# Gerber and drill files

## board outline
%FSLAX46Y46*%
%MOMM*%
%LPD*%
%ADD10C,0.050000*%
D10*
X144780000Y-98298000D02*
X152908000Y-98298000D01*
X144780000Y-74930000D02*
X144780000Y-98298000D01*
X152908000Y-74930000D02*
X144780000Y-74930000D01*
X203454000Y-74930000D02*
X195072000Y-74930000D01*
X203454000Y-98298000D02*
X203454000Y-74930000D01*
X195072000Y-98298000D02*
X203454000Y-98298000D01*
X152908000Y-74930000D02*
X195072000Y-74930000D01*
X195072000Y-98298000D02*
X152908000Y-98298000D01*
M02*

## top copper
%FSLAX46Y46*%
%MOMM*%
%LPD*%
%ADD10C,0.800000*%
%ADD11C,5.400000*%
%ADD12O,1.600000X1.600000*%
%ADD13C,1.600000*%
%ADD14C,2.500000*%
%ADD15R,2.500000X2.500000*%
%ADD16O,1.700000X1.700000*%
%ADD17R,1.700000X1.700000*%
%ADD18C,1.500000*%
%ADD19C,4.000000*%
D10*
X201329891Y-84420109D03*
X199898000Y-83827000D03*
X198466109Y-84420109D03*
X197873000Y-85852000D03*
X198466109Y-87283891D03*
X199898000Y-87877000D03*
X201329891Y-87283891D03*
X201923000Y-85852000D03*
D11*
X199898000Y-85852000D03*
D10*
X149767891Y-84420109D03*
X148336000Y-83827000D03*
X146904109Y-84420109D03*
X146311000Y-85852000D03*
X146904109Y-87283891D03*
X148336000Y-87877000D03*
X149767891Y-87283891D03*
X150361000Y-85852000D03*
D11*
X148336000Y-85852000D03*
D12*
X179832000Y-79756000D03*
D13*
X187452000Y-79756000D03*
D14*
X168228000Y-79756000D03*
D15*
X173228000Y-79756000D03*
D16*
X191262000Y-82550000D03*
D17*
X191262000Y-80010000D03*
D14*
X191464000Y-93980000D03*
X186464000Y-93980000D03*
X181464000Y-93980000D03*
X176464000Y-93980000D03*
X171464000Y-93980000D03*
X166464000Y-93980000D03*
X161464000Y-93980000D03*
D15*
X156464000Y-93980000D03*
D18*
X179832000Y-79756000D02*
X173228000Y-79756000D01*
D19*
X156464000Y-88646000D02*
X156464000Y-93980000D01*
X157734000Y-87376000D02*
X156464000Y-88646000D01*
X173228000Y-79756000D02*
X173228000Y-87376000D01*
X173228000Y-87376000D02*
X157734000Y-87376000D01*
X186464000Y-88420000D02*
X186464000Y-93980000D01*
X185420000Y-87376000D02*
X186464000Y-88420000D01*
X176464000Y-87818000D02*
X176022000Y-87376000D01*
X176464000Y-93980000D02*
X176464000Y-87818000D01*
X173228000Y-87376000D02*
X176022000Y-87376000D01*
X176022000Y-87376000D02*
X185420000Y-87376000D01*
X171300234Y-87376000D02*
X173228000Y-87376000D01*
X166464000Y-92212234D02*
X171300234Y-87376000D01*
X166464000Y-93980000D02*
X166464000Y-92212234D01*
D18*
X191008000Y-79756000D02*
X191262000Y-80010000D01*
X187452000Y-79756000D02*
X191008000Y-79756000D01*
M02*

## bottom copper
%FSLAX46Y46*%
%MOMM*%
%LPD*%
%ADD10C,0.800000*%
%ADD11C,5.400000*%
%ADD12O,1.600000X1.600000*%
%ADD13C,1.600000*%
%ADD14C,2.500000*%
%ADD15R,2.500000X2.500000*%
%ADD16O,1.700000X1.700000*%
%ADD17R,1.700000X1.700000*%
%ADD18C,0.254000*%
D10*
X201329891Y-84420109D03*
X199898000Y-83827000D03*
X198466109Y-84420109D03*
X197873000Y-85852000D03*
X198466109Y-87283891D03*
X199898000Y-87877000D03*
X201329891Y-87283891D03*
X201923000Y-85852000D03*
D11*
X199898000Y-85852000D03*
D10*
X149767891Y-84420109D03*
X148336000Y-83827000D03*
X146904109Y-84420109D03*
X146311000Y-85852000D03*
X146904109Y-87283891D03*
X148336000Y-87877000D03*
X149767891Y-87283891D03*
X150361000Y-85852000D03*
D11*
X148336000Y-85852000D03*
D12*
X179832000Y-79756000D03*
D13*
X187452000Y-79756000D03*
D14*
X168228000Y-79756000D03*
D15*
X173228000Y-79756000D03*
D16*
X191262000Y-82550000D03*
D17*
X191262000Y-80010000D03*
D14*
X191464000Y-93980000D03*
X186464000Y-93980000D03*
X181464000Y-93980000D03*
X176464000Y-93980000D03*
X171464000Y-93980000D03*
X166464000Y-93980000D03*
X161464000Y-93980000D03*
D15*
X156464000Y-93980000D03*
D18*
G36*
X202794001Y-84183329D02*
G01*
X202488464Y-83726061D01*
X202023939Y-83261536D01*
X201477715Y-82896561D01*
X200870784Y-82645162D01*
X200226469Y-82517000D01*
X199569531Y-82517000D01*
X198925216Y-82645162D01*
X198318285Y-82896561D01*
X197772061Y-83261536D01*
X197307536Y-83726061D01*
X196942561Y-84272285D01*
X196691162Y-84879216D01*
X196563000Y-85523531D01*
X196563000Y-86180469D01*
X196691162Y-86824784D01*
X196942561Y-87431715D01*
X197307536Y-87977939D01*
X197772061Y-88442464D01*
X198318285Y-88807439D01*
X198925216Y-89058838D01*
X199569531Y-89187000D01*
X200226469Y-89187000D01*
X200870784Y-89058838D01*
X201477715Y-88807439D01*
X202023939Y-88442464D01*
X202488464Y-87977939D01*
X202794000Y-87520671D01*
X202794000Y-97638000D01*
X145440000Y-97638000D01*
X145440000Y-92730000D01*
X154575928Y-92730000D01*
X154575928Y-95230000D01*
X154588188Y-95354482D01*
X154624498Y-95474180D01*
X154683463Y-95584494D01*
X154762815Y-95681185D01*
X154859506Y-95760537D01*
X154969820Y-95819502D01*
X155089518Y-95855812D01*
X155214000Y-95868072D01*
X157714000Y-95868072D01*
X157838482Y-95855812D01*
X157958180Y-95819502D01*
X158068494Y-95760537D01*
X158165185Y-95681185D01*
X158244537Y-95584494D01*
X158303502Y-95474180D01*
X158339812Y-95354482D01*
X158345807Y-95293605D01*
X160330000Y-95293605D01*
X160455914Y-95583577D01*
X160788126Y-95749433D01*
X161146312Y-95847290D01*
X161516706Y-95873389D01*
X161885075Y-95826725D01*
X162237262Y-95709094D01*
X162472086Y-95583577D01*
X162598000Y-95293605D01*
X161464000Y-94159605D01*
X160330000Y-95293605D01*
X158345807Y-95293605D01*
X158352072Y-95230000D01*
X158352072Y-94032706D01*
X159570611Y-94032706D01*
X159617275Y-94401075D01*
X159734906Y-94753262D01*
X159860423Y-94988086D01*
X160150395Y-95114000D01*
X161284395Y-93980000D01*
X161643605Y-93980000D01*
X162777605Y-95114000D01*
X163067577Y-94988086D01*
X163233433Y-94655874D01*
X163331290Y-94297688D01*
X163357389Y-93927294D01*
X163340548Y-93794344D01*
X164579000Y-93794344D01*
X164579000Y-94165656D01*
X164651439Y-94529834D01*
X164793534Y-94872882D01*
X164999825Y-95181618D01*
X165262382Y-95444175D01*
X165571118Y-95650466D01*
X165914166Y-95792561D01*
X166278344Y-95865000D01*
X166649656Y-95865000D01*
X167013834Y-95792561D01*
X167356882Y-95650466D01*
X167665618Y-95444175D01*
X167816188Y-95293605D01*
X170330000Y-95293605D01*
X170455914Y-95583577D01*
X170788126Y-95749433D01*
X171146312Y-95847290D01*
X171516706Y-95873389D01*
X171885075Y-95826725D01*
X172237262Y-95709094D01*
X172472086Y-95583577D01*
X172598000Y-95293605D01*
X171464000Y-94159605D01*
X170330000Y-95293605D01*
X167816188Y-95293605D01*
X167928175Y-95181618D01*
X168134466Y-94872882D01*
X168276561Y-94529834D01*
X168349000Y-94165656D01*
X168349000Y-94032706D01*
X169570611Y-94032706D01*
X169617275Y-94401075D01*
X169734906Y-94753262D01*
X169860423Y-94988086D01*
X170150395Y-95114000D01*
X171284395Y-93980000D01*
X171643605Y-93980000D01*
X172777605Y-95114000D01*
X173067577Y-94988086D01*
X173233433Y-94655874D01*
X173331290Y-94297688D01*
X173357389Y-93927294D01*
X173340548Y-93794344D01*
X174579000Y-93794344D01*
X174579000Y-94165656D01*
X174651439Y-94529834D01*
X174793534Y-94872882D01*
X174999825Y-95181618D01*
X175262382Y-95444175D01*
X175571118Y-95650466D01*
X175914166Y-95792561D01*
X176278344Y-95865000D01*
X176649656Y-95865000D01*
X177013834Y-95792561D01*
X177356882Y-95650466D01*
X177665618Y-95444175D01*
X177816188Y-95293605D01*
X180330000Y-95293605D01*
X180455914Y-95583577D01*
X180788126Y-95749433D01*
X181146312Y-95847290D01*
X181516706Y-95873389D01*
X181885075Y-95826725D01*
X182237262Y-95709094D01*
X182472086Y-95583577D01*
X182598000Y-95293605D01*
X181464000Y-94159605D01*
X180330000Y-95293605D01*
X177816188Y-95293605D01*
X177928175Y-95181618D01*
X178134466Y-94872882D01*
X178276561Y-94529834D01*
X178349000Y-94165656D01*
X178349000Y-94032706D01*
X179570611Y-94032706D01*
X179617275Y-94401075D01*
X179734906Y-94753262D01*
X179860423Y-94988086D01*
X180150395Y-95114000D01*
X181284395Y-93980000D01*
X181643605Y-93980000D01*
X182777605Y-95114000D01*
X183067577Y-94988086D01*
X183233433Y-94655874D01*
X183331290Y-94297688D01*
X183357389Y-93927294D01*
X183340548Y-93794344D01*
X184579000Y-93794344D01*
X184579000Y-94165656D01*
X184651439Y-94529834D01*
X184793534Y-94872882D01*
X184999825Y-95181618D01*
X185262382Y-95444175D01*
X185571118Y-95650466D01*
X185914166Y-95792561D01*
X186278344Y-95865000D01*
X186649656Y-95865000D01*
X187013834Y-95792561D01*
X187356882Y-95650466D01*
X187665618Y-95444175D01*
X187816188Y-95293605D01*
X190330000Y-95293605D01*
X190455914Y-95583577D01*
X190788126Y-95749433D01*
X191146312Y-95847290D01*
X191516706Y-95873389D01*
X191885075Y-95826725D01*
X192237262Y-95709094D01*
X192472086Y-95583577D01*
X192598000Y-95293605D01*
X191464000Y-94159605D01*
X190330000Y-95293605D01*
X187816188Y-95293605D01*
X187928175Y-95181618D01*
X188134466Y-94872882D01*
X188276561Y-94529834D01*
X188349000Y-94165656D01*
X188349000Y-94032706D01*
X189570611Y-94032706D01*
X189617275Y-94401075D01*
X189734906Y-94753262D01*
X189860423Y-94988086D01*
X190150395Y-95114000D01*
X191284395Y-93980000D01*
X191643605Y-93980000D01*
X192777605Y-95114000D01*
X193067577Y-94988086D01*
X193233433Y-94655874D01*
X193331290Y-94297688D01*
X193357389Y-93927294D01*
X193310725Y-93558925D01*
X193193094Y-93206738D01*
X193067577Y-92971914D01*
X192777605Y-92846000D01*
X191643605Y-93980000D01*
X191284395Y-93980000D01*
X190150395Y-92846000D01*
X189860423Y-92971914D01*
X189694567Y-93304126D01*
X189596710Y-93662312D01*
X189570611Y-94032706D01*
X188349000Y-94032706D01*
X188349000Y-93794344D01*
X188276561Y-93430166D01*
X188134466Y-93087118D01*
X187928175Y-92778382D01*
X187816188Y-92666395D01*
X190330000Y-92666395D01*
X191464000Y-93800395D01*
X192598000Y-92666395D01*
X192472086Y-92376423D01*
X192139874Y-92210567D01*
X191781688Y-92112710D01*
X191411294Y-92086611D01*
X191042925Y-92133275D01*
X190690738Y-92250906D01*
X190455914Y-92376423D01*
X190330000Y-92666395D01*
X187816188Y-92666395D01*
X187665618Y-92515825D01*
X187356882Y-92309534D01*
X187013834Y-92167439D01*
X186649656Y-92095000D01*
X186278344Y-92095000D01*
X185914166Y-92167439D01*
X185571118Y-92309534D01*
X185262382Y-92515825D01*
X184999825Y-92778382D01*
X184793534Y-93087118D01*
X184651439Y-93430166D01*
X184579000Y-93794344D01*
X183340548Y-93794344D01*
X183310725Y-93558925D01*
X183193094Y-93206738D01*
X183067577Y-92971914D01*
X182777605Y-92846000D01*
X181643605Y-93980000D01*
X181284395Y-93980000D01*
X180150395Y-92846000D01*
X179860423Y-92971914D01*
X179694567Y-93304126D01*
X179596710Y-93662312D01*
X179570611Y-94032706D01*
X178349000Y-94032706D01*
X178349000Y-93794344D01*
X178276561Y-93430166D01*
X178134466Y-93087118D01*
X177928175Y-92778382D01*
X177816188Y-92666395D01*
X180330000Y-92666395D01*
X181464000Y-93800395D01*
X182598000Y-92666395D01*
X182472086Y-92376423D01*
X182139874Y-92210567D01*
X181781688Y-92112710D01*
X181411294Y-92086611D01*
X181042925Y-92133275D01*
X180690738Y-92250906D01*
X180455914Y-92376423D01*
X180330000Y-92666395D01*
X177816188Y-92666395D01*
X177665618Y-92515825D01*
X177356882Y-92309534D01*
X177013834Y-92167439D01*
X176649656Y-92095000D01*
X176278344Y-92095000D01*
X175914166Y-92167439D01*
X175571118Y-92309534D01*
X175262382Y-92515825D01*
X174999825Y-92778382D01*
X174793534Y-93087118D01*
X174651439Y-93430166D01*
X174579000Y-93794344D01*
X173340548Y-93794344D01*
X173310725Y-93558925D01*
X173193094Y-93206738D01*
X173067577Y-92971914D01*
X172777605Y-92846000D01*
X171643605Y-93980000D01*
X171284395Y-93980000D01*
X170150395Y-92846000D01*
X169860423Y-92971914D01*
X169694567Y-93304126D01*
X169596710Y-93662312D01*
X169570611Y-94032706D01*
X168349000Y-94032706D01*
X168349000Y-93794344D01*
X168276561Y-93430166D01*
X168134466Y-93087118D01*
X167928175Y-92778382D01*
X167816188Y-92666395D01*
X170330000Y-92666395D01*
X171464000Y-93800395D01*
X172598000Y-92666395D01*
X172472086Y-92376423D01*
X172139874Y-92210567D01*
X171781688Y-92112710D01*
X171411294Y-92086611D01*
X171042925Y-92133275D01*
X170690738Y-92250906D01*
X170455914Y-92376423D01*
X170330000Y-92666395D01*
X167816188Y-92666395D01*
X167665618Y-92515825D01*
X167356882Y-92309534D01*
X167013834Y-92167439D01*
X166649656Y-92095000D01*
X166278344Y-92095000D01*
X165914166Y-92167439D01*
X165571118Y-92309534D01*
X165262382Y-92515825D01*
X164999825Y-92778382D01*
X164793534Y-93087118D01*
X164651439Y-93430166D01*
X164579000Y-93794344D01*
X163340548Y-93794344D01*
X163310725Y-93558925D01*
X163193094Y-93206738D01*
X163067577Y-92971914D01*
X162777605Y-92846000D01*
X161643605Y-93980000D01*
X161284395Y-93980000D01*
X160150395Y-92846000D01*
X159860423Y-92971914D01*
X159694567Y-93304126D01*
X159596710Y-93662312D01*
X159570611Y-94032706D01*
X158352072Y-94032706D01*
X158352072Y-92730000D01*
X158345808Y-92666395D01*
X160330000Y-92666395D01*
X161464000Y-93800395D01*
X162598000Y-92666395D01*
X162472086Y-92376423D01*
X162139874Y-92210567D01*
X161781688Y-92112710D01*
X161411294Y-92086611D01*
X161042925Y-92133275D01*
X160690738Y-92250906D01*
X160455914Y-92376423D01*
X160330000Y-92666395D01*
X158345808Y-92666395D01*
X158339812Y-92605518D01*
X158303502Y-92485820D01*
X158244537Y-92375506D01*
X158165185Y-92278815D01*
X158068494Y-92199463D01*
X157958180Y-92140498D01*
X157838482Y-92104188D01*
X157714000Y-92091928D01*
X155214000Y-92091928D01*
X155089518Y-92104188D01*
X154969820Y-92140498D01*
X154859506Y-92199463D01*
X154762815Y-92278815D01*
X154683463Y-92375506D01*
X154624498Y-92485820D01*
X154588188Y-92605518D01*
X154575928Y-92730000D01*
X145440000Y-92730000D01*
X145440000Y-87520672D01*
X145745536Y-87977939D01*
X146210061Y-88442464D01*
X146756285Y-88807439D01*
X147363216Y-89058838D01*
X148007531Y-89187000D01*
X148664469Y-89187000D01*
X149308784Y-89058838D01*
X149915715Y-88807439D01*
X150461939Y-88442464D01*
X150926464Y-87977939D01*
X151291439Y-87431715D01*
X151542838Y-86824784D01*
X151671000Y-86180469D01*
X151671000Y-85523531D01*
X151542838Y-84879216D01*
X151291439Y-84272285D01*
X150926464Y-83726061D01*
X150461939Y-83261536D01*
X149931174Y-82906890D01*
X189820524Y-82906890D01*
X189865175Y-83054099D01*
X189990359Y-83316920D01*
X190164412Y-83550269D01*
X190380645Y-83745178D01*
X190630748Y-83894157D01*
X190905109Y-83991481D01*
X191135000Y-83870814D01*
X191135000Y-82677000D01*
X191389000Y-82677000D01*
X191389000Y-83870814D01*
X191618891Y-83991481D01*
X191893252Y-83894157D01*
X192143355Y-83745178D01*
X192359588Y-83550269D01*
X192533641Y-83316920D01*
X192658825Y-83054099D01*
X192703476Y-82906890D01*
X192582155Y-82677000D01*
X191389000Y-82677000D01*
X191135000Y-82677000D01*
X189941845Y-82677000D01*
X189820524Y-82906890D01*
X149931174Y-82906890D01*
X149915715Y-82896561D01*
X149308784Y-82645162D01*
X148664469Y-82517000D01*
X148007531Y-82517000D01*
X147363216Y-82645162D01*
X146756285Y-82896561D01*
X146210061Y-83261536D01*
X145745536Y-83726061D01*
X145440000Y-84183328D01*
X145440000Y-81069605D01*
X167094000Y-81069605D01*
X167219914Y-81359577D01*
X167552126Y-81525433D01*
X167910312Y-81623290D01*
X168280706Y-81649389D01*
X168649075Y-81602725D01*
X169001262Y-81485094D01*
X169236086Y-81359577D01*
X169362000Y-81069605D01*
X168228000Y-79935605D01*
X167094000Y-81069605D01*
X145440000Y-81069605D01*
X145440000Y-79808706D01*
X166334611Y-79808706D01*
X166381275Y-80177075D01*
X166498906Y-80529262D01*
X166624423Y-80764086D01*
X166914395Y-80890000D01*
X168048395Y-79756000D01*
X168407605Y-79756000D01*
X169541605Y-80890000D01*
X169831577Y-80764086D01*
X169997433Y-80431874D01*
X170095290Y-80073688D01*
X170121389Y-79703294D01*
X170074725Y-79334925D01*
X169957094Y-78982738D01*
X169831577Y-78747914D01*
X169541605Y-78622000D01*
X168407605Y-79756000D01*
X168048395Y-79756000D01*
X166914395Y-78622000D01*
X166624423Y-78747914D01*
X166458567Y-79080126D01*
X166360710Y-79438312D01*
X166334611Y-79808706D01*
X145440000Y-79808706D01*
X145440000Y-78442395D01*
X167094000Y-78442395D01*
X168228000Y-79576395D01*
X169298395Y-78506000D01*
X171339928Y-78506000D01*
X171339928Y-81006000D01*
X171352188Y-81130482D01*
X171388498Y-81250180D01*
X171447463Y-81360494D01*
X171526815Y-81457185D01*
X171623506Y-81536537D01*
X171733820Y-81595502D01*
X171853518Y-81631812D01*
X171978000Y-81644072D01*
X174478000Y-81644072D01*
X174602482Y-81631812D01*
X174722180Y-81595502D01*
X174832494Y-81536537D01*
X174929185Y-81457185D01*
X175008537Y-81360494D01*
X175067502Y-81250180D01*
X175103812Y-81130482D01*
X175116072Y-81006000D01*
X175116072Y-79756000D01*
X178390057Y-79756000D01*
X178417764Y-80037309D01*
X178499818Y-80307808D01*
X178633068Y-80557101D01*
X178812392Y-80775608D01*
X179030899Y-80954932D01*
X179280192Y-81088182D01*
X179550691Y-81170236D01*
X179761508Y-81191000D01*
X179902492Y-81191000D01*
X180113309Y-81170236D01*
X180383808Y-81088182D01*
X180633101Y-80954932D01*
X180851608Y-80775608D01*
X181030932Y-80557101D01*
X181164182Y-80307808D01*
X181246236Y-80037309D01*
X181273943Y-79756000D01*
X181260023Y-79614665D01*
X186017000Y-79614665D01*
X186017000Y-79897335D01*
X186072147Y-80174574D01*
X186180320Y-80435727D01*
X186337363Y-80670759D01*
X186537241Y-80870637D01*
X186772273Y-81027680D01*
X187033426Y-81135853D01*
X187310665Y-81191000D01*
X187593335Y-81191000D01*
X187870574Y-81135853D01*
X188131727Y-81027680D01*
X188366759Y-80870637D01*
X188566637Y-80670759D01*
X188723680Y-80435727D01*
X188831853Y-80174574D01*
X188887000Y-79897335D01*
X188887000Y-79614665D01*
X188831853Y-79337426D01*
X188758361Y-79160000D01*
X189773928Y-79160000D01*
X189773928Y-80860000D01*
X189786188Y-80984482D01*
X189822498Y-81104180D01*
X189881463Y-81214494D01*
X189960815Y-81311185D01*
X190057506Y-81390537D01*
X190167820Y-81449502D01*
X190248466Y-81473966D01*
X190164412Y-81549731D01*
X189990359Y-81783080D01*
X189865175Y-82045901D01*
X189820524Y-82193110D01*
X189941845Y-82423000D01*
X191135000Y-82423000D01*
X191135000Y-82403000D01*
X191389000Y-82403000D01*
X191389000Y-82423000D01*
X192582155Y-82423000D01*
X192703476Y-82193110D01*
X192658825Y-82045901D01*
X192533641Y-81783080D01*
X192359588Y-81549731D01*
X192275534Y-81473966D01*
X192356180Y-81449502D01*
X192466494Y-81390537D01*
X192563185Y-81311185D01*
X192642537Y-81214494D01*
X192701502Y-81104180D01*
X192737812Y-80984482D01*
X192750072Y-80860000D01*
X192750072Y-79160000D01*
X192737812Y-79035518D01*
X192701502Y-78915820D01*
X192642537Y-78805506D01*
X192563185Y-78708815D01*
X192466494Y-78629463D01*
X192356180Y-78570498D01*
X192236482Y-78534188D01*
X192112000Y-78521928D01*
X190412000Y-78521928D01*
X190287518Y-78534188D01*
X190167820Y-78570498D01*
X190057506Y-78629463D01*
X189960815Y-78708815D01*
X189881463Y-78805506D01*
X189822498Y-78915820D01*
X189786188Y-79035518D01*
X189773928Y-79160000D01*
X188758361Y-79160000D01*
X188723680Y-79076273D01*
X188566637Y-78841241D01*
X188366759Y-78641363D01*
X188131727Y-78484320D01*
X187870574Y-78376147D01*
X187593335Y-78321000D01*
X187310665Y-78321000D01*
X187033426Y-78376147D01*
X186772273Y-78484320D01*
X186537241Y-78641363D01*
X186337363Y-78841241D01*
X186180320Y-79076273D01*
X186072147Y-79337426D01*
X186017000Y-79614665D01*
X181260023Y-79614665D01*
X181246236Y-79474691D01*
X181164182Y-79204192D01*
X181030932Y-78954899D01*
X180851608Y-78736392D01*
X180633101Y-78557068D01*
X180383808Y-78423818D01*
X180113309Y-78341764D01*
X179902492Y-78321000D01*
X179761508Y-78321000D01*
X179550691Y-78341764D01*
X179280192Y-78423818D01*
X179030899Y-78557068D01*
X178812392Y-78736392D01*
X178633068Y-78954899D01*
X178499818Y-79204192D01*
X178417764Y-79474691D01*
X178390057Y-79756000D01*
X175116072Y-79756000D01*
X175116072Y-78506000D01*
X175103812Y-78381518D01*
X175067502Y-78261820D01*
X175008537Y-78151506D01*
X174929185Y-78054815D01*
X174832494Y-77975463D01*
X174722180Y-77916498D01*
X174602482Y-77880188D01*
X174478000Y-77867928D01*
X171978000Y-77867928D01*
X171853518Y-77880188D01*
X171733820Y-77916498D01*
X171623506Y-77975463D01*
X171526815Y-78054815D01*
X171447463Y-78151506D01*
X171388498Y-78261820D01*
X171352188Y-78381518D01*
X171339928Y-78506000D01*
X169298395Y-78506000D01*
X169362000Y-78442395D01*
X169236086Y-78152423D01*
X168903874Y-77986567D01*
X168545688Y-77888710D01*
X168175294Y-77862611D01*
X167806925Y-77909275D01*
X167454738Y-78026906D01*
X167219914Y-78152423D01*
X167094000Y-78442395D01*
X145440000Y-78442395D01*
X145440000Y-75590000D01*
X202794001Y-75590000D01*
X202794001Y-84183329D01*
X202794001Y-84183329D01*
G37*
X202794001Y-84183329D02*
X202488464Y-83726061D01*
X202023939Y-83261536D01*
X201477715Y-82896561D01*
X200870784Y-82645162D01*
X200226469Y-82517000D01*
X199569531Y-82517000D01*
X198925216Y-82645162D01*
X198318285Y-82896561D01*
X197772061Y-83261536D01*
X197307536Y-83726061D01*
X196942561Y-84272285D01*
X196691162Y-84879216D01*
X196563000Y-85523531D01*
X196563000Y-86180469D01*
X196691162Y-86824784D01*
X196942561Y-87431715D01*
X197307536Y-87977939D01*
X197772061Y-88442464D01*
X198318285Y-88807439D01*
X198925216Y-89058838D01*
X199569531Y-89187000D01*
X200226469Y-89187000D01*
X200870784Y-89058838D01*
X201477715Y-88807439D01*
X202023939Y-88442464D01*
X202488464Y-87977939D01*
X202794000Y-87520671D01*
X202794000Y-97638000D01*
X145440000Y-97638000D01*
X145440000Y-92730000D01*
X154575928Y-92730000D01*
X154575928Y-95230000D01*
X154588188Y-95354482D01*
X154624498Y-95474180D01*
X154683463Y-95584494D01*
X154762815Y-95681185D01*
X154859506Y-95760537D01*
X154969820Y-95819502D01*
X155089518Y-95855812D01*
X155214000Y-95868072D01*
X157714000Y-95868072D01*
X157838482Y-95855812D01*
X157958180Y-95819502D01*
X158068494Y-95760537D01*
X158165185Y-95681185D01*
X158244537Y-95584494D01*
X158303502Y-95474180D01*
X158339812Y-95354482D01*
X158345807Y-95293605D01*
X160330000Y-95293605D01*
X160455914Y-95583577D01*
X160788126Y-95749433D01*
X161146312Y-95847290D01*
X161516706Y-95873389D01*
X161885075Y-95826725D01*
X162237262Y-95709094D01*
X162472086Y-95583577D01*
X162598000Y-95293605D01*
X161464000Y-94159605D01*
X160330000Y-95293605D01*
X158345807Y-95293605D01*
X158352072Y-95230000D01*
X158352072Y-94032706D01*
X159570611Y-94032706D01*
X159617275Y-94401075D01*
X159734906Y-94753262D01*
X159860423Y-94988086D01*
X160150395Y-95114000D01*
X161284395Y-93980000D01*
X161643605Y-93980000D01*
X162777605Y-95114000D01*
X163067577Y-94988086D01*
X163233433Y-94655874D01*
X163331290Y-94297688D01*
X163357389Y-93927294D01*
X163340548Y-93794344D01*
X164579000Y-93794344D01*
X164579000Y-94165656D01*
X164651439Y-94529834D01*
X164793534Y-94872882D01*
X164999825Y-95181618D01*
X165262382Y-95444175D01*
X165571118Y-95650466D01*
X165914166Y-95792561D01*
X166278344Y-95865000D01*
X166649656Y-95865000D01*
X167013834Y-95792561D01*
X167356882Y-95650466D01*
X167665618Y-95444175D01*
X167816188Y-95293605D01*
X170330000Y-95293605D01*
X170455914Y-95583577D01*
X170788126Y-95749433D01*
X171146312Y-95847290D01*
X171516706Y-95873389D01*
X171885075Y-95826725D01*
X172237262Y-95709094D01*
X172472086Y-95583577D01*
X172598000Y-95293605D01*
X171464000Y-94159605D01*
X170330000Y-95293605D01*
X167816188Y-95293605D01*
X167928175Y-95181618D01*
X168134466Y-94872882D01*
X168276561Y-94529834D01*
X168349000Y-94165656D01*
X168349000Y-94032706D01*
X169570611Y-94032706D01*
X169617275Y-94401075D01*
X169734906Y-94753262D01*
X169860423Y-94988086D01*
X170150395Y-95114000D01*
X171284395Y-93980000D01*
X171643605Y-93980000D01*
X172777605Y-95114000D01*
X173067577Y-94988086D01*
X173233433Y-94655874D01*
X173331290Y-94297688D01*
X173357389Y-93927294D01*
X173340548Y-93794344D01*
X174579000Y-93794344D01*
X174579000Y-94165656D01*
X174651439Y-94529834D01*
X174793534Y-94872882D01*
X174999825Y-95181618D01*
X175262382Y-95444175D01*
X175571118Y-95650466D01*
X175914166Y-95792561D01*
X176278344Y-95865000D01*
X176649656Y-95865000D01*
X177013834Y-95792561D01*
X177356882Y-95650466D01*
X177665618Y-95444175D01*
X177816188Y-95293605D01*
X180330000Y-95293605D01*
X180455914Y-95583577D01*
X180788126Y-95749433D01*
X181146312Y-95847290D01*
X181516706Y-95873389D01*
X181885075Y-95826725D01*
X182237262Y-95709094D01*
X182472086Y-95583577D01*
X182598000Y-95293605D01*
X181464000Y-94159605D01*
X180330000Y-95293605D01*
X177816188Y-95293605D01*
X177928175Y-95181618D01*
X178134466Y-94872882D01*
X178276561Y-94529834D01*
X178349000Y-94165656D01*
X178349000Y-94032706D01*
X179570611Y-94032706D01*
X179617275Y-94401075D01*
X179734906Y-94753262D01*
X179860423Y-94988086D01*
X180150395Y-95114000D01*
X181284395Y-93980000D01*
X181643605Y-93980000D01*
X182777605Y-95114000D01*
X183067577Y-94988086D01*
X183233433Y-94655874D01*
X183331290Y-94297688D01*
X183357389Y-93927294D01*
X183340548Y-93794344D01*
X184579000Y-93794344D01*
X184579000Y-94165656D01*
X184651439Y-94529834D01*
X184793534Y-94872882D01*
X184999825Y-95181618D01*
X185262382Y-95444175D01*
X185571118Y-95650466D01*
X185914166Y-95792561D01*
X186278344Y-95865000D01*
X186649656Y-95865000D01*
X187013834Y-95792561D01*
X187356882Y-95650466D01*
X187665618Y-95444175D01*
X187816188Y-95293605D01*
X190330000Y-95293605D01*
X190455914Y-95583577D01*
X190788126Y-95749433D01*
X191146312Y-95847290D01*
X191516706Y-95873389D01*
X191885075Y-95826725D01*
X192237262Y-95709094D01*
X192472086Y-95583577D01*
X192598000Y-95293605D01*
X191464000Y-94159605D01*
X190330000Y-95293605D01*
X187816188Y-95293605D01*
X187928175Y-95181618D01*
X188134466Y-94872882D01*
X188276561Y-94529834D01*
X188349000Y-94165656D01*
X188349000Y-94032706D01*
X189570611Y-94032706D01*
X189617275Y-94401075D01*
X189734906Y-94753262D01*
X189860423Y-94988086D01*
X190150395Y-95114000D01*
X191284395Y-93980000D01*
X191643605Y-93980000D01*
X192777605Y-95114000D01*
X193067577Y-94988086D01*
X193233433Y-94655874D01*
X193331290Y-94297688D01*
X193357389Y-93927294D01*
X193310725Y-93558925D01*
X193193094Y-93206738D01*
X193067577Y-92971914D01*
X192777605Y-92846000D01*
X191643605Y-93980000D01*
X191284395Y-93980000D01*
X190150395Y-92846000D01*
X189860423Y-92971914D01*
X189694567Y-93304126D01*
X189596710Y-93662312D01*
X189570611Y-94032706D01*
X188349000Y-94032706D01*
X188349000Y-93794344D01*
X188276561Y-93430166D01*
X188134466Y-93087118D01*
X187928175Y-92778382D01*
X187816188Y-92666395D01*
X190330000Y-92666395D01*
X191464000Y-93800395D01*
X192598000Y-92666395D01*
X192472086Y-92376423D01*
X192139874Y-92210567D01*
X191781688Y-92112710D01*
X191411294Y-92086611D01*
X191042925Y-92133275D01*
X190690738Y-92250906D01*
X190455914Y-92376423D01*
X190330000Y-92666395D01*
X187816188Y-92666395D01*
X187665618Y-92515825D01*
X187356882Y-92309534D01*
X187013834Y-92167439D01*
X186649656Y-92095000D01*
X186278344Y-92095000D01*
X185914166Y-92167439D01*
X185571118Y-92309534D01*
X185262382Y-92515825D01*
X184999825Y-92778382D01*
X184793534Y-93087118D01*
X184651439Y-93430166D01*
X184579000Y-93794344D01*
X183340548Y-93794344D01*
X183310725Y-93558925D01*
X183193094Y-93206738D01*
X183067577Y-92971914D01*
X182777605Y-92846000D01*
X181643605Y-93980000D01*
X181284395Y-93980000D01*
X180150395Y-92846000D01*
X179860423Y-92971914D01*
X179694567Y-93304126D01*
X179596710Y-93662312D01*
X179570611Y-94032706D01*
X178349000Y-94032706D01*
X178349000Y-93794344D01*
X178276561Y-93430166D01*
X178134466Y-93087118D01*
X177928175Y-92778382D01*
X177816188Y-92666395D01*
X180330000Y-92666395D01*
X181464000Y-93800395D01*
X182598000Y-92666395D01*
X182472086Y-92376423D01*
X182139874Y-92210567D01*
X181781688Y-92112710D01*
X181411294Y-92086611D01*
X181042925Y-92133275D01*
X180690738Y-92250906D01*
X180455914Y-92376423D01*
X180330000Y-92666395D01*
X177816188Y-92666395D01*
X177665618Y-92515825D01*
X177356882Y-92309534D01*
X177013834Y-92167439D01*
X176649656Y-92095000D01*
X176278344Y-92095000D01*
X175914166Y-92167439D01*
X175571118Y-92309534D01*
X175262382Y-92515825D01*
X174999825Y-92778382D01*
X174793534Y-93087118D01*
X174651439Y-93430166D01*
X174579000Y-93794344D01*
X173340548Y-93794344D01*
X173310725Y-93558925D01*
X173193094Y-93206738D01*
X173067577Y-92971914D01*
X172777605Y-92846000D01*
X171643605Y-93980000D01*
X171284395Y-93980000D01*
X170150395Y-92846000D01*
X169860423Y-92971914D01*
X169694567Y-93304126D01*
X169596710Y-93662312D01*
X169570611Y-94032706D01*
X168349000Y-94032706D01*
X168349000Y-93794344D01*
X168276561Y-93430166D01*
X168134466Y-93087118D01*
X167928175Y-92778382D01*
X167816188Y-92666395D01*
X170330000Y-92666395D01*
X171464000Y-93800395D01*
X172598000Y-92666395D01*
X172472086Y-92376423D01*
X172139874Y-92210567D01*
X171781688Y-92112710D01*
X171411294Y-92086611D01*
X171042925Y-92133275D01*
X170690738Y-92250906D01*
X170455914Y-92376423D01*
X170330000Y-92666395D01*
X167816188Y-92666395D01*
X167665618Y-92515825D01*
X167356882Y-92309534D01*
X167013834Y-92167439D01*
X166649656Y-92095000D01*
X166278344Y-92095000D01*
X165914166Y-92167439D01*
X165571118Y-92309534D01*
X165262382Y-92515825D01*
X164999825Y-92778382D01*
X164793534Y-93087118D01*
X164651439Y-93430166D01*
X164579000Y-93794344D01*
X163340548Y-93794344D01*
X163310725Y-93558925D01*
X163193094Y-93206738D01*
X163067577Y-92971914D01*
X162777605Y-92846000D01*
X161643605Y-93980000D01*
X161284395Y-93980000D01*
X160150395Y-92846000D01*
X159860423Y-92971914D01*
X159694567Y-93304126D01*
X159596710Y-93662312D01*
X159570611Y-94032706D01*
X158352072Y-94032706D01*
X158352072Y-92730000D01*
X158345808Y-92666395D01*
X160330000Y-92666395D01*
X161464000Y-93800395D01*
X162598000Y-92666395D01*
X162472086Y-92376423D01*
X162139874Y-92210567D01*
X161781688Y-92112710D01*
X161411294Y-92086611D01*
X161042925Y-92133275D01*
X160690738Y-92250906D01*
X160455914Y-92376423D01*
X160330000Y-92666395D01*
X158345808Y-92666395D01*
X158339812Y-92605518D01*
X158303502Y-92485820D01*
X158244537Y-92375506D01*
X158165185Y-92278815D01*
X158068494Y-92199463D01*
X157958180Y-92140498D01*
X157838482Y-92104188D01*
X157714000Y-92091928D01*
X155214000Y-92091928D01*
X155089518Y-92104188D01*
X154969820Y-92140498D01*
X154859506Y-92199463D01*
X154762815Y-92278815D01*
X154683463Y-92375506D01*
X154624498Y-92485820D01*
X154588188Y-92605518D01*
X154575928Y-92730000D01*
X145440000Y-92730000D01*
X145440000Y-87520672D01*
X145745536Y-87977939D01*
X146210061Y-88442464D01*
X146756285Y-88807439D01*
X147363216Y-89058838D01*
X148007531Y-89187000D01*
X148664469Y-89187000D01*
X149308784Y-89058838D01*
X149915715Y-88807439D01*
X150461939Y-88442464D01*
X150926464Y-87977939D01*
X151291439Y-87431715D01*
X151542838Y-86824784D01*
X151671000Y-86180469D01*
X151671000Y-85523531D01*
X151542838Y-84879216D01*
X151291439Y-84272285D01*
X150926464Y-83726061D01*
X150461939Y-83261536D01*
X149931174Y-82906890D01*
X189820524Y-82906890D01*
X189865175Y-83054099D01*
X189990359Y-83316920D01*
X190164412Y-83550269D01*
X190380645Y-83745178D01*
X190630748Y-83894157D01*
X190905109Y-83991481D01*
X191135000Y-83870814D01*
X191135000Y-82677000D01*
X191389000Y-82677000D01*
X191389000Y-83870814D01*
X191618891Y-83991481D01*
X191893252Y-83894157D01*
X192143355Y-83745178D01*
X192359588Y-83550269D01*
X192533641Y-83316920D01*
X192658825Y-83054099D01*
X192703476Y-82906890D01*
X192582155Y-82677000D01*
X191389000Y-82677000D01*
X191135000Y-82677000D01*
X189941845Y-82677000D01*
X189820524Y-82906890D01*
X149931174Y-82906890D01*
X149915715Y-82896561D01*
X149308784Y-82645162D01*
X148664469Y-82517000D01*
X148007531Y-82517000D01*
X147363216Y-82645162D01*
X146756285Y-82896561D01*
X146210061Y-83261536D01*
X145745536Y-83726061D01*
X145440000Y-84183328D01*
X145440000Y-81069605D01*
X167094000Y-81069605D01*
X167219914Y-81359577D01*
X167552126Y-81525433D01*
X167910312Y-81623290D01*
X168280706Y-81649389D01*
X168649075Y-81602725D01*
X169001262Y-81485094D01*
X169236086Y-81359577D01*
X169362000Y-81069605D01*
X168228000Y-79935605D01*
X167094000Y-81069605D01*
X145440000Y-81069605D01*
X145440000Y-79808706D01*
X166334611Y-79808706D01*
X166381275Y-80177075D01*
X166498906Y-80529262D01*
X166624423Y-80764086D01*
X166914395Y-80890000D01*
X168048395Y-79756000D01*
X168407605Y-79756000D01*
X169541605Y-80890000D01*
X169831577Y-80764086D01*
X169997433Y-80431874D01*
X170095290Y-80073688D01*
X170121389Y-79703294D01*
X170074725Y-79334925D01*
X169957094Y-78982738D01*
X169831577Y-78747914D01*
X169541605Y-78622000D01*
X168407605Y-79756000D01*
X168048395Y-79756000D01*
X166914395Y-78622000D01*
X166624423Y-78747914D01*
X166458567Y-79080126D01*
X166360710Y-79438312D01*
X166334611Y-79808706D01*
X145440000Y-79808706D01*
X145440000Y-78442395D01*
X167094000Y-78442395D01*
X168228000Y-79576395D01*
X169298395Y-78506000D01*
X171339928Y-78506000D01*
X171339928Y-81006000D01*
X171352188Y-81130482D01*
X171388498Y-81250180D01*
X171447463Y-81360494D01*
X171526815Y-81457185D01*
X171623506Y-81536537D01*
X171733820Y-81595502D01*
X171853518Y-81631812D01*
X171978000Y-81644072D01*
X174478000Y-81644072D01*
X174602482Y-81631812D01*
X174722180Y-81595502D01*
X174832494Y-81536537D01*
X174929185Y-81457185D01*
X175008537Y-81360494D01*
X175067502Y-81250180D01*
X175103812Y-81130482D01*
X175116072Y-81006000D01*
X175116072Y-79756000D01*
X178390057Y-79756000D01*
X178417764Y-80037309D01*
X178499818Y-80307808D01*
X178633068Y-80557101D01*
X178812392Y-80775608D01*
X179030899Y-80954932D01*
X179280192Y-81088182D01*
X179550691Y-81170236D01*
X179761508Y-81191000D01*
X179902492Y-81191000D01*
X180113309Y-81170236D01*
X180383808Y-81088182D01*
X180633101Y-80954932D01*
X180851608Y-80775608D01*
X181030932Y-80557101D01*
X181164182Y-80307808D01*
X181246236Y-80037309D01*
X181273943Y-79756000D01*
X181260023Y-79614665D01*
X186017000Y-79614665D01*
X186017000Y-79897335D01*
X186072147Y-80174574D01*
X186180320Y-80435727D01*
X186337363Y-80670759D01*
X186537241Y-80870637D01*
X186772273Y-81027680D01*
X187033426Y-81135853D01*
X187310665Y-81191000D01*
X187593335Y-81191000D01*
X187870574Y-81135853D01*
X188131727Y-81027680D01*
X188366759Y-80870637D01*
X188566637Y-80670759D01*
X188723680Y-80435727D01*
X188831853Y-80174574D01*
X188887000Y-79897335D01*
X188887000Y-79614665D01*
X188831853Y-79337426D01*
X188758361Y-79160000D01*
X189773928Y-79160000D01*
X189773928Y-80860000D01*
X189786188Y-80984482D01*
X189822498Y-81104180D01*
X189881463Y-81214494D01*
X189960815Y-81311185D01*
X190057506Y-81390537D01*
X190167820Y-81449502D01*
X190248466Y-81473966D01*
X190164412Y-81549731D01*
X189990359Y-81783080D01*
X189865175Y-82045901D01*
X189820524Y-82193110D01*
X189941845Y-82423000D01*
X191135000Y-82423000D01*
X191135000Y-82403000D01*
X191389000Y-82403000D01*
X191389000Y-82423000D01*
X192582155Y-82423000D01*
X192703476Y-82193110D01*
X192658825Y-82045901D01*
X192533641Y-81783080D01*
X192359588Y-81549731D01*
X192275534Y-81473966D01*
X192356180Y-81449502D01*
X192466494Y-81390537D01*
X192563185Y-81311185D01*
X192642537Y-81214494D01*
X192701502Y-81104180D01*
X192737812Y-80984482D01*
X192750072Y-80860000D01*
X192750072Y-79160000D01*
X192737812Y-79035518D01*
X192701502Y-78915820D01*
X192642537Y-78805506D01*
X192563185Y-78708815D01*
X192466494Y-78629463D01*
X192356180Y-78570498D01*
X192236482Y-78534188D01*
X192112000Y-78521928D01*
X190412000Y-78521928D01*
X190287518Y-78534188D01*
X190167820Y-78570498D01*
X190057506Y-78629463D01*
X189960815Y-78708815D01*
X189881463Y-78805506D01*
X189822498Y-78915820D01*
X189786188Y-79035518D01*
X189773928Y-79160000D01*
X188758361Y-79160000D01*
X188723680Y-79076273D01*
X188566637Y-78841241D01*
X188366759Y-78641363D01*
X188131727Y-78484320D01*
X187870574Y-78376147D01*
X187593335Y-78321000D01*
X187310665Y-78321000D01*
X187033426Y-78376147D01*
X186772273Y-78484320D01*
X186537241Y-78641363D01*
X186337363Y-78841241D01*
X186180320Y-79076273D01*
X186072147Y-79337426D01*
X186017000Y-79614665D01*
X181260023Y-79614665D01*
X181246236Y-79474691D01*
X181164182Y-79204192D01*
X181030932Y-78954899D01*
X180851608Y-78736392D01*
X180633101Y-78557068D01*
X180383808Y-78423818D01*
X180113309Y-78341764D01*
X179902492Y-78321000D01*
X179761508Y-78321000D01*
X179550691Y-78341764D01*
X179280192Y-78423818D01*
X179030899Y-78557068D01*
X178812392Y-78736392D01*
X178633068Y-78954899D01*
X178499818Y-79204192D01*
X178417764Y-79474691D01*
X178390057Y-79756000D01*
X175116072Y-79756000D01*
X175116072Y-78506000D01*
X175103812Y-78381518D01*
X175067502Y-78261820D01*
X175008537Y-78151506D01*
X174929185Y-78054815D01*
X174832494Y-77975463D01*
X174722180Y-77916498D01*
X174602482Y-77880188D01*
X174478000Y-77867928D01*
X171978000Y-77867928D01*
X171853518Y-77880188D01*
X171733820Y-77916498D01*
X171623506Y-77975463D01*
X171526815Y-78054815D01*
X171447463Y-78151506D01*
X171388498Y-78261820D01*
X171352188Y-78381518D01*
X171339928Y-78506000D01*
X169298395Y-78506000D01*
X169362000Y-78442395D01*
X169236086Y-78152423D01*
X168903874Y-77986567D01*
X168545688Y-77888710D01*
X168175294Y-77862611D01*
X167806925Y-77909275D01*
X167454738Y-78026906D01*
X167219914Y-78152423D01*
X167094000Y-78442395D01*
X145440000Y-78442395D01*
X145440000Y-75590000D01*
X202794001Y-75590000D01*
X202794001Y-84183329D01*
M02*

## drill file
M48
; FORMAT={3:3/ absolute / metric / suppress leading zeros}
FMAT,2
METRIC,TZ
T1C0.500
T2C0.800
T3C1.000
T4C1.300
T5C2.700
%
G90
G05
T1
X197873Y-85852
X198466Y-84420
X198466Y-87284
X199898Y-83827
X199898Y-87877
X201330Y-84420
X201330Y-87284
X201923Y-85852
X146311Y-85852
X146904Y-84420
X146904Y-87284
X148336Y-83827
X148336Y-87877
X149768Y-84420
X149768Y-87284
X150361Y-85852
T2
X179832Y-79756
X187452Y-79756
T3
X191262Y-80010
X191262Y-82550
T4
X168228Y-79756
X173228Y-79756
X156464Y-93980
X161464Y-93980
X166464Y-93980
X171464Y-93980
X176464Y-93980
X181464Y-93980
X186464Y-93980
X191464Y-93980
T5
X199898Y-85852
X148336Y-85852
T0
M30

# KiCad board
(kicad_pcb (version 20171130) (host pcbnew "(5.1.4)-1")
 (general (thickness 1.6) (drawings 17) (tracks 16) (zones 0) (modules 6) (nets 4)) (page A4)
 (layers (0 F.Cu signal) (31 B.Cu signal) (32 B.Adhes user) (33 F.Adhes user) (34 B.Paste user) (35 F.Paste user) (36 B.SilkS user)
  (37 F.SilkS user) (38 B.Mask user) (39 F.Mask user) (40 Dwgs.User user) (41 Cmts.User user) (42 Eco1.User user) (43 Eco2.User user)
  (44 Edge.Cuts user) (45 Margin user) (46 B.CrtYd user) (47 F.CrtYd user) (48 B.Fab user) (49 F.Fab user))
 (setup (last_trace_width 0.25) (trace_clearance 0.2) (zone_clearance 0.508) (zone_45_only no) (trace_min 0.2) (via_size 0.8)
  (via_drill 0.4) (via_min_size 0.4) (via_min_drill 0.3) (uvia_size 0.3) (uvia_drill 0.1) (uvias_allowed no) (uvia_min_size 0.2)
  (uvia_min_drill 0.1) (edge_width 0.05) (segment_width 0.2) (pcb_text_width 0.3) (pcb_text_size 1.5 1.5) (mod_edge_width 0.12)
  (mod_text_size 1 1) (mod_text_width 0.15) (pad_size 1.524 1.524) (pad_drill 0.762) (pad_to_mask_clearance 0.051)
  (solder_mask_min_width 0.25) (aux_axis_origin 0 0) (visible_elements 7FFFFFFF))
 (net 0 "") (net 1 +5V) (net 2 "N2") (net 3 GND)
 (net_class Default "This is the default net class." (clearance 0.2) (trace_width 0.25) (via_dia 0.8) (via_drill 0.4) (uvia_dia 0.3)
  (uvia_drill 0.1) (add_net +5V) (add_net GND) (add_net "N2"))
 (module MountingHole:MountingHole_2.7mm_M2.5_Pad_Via (layer F.Cu) (at 199.898 85.852)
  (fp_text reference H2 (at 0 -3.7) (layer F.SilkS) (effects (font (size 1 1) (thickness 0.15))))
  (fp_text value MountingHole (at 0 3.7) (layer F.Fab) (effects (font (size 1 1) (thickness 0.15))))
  (pad 1 thru_hole circle (at 1.431891 -1.431891) (size 0.8 0.8) (drill 0.5) (layers *.Cu *.Mask))
  (pad 1 thru_hole circle (at 0 -2.025) (size 0.8 0.8) (drill 0.5) (layers *.Cu *.Mask))
  (pad 1 thru_hole circle (at -1.431891 -1.431891) (size 0.8 0.8) (drill 0.5) (layers *.Cu *.Mask))
  (pad 1 thru_hole circle (at -2.025 0) (size 0.8 0.8) (drill 0.5) (layers *.Cu *.Mask))
  (pad 1 thru_hole circle (at -1.431891 1.431891) (size 0.8 0.8) (drill 0.5) (layers *.Cu *.Mask))
  (pad 1 thru_hole circle (at 0 2.025) (size 0.8 0.8) (drill 0.5) (layers *.Cu *.Mask))
  (pad 1 thru_hole circle (at 1.431891 1.431891) (size 0.8 0.8) (drill 0.5) (layers *.Cu *.Mask))
  (pad 1 thru_hole circle (at 2.025 0) (size 0.8 0.8) (drill 0.5) (layers *.Cu *.Mask))
  (pad 1 thru_hole circle (at 0 0) (size 5.4 5.4) (drill 2.7) (layers *.Cu *.Mask)))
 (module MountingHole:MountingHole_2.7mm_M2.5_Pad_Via (layer F.Cu) (at 148.336 85.852)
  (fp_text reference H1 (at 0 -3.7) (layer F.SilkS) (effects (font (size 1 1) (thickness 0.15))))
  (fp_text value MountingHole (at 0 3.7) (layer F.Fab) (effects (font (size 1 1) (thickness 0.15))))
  (pad 1 thru_hole circle (at 1.431891 -1.431891) (size 0.8 0.8) (drill 0.5) (layers *.Cu *.Mask))
  (pad 1 thru_hole circle (at 0 -2.025) (size 0.8 0.8) (drill 0.5) (layers *.Cu *.Mask))
  (pad 1 thru_hole circle (at -1.431891 -1.431891) (size 0.8 0.8) (drill 0.5) (layers *.Cu *.Mask))
  (pad 1 thru_hole circle (at -2.025 0) (size 0.8 0.8) (drill 0.5) (layers *.Cu *.Mask))
  (pad 1 thru_hole circle (at -1.431891 1.431891) (size 0.8 0.8) (drill 0.5) (layers *.Cu *.Mask))
  (pad 1 thru_hole circle (at 0 2.025) (size 0.8 0.8) (drill 0.5) (layers *.Cu *.Mask))
  (pad 1 thru_hole circle (at 1.431891 1.431891) (size 0.8 0.8) (drill 0.5) (layers *.Cu *.Mask))
  (pad 1 thru_hole circle (at 2.025 0) (size 0.8 0.8) (drill 0.5) (layers *.Cu *.Mask))
  (pad 1 thru_hole circle (at 0 0) (size 5.4 5.4) (drill 2.7) (layers *.Cu *.Mask)))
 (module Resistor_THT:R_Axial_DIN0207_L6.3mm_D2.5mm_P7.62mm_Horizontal (layer F.Cu) (at 187.452 79.756 180)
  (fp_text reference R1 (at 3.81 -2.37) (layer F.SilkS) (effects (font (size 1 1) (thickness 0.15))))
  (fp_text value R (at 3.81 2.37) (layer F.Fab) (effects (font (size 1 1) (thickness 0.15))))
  (pad 2 thru_hole oval (at 7.62 0 180) (size 1.6 1.6) (drill 0.8) (layers *.Cu *.Mask) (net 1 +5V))
  (pad 1 thru_hole circle (at 0 0 180) (size 1.6 1.6) (drill 0.8) (layers *.Cu *.Mask) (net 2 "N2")))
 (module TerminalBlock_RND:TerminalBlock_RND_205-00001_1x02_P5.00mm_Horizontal (layer F.Cu) (at 173.228 79.756 180)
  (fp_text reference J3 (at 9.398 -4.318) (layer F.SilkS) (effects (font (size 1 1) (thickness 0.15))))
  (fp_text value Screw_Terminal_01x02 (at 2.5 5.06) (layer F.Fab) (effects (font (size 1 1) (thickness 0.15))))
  (pad 2 thru_hole circle (at 5 0 180) (size 2.5 2.5) (drill 1.3) (layers *.Cu *.Mask) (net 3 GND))
  (pad 1 thru_hole rect (at 0 0 180) (size 2.5 2.5) (drill 1.3) (layers *.Cu *.Mask) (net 1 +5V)))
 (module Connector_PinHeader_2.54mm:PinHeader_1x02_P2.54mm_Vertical (layer F.Cu) (at 191.262 80.01)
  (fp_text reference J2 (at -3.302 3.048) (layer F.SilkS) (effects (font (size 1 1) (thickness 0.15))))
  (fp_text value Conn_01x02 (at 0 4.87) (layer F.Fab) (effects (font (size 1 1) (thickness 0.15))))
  (pad 2 thru_hole oval (at 0 2.54) (size 1.7 1.7) (drill 1) (layers *.Cu *.Mask) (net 3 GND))
  (pad 1 thru_hole rect (at 0 0) (size 1.7 1.7) (drill 1) (layers *.Cu *.Mask) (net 2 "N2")))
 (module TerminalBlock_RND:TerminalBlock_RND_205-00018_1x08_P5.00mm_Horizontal (layer F.Cu) (at 156.464 93.98)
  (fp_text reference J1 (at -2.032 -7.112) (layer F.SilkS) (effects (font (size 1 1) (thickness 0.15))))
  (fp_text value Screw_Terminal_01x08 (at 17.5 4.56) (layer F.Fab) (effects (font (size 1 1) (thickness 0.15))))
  (pad 8 thru_hole circle (at 35 0) (size 2.5 2.5) (drill 1.3) (layers *.Cu *.Mask) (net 3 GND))
  (pad 7 thru_hole circle (at 30 0) (size 2.5 2.5) (drill 1.3) (layers *.Cu *.Mask) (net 1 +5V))
  (pad 6 thru_hole circle (at 25 0) (size 2.5 2.5) (drill 1.3) (layers *.Cu *.Mask) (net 3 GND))
  (pad 5 thru_hole circle (at 20 0) (size 2.5 2.5) (drill 1.3) (layers *.Cu *.Mask) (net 1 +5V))
  (pad 4 thru_hole circle (at 15 0) (size 2.5 2.5) (drill 1.3) (layers *.Cu *.Mask) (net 3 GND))
  (pad 3 thru_hole circle (at 10 0) (size 2.5 2.5) (drill 1.3) (layers *.Cu *.Mask) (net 1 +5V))
  (pad 2 thru_hole circle (at 5 0) (size 2.5 2.5) (drill 1.3) (layers *.Cu *.Mask) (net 3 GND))
  (pad 1 thru_hole rect (at 0 0) (size 2.5 2.5) (drill 1.3) (layers *.Cu *.Mask) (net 1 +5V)))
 (gr_line (start 144.78 98.298) (end 152.908 98.298) (layer Edge.Cuts) (width 0.05))
 (gr_line (start 144.78 74.93) (end 144.78 98.298) (layer Edge.Cuts) (width 0.05))
 (gr_line (start 152.908 74.93) (end 144.78 74.93) (layer Edge.Cuts) (width 0.05))
 (gr_line (start 203.454 74.93) (end 195.072 74.93) (layer Edge.Cuts) (width 0.05))
 (gr_line (start 203.454 98.298) (end 203.454 74.93) (layer Edge.Cuts) (width 0.05))
 (gr_line (start 195.072 98.298) (end 203.454 98.298) (layer Edge.Cuts) (width 0.05))
 (gr_line (start 152.908 74.93) (end 195.072 74.93) (layer Edge.Cuts) (width 0.05))
 (gr_line (start 195.072 98.298) (end 152.908 98.298) (layer Edge.Cuts) (width 0.05))
 (segment (start 179.832 79.756) (end 173.228 79.756) (width 1.5) (layer F.Cu) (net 1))
 (segment (start 156.464 88.646) (end 156.464 93.98) (width 4) (layer F.Cu) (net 1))
 (segment (start 157.734 87.376) (end 156.464 88.646) (width 4) (layer F.Cu) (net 1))
 (segment (start 173.228 79.756) (end 173.228 87.376) (width 4) (layer F.Cu) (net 1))
 (segment (start 173.228 87.376) (end 157.734 87.376) (width 4) (layer F.Cu) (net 1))
 (segment (start 186.464 88.42) (end 186.464 93.98) (width 4) (layer F.Cu) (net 1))
 (segment (start 185.42 87.376) (end 186.464 88.42) (width 4) (layer F.Cu) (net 1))
 (segment (start 176.464 87.818) (end 176.022 87.376) (width 4) (layer F.Cu) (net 1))
 (segment (start 176.464 93.98) (end 176.464 87.818) (width 4) (layer F.Cu) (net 1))
 (segment (start 173.228 87.376) (end 176.022 87.376) (width 4) (layer F.Cu) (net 1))
 (segment (start 176.022 87.376) (end 185.42 87.376) (width 4) (layer F.Cu) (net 1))
 (segment (start 171.300234 87.376) (end 173.228 87.376) (width 4) (layer F.Cu) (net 1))
 (segment (start 166.464 92.212234) (end 171.300234 87.376) (width 4) (layer F.Cu) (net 1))
 (segment (start 166.464 93.98) (end 166.464 92.212234) (width 4) (layer F.Cu) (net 1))
 (segment (start 191.008 79.756) (end 191.262 80.01) (width 1.5) (layer F.Cu) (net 2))
 (segment (start 187.452 79.756) (end 191.008 79.756) (width 1.5) (layer F.Cu) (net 2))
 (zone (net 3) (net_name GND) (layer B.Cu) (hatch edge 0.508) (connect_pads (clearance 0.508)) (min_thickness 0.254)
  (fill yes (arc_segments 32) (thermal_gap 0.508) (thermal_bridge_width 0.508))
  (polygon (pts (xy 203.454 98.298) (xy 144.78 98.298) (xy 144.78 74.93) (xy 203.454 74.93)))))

